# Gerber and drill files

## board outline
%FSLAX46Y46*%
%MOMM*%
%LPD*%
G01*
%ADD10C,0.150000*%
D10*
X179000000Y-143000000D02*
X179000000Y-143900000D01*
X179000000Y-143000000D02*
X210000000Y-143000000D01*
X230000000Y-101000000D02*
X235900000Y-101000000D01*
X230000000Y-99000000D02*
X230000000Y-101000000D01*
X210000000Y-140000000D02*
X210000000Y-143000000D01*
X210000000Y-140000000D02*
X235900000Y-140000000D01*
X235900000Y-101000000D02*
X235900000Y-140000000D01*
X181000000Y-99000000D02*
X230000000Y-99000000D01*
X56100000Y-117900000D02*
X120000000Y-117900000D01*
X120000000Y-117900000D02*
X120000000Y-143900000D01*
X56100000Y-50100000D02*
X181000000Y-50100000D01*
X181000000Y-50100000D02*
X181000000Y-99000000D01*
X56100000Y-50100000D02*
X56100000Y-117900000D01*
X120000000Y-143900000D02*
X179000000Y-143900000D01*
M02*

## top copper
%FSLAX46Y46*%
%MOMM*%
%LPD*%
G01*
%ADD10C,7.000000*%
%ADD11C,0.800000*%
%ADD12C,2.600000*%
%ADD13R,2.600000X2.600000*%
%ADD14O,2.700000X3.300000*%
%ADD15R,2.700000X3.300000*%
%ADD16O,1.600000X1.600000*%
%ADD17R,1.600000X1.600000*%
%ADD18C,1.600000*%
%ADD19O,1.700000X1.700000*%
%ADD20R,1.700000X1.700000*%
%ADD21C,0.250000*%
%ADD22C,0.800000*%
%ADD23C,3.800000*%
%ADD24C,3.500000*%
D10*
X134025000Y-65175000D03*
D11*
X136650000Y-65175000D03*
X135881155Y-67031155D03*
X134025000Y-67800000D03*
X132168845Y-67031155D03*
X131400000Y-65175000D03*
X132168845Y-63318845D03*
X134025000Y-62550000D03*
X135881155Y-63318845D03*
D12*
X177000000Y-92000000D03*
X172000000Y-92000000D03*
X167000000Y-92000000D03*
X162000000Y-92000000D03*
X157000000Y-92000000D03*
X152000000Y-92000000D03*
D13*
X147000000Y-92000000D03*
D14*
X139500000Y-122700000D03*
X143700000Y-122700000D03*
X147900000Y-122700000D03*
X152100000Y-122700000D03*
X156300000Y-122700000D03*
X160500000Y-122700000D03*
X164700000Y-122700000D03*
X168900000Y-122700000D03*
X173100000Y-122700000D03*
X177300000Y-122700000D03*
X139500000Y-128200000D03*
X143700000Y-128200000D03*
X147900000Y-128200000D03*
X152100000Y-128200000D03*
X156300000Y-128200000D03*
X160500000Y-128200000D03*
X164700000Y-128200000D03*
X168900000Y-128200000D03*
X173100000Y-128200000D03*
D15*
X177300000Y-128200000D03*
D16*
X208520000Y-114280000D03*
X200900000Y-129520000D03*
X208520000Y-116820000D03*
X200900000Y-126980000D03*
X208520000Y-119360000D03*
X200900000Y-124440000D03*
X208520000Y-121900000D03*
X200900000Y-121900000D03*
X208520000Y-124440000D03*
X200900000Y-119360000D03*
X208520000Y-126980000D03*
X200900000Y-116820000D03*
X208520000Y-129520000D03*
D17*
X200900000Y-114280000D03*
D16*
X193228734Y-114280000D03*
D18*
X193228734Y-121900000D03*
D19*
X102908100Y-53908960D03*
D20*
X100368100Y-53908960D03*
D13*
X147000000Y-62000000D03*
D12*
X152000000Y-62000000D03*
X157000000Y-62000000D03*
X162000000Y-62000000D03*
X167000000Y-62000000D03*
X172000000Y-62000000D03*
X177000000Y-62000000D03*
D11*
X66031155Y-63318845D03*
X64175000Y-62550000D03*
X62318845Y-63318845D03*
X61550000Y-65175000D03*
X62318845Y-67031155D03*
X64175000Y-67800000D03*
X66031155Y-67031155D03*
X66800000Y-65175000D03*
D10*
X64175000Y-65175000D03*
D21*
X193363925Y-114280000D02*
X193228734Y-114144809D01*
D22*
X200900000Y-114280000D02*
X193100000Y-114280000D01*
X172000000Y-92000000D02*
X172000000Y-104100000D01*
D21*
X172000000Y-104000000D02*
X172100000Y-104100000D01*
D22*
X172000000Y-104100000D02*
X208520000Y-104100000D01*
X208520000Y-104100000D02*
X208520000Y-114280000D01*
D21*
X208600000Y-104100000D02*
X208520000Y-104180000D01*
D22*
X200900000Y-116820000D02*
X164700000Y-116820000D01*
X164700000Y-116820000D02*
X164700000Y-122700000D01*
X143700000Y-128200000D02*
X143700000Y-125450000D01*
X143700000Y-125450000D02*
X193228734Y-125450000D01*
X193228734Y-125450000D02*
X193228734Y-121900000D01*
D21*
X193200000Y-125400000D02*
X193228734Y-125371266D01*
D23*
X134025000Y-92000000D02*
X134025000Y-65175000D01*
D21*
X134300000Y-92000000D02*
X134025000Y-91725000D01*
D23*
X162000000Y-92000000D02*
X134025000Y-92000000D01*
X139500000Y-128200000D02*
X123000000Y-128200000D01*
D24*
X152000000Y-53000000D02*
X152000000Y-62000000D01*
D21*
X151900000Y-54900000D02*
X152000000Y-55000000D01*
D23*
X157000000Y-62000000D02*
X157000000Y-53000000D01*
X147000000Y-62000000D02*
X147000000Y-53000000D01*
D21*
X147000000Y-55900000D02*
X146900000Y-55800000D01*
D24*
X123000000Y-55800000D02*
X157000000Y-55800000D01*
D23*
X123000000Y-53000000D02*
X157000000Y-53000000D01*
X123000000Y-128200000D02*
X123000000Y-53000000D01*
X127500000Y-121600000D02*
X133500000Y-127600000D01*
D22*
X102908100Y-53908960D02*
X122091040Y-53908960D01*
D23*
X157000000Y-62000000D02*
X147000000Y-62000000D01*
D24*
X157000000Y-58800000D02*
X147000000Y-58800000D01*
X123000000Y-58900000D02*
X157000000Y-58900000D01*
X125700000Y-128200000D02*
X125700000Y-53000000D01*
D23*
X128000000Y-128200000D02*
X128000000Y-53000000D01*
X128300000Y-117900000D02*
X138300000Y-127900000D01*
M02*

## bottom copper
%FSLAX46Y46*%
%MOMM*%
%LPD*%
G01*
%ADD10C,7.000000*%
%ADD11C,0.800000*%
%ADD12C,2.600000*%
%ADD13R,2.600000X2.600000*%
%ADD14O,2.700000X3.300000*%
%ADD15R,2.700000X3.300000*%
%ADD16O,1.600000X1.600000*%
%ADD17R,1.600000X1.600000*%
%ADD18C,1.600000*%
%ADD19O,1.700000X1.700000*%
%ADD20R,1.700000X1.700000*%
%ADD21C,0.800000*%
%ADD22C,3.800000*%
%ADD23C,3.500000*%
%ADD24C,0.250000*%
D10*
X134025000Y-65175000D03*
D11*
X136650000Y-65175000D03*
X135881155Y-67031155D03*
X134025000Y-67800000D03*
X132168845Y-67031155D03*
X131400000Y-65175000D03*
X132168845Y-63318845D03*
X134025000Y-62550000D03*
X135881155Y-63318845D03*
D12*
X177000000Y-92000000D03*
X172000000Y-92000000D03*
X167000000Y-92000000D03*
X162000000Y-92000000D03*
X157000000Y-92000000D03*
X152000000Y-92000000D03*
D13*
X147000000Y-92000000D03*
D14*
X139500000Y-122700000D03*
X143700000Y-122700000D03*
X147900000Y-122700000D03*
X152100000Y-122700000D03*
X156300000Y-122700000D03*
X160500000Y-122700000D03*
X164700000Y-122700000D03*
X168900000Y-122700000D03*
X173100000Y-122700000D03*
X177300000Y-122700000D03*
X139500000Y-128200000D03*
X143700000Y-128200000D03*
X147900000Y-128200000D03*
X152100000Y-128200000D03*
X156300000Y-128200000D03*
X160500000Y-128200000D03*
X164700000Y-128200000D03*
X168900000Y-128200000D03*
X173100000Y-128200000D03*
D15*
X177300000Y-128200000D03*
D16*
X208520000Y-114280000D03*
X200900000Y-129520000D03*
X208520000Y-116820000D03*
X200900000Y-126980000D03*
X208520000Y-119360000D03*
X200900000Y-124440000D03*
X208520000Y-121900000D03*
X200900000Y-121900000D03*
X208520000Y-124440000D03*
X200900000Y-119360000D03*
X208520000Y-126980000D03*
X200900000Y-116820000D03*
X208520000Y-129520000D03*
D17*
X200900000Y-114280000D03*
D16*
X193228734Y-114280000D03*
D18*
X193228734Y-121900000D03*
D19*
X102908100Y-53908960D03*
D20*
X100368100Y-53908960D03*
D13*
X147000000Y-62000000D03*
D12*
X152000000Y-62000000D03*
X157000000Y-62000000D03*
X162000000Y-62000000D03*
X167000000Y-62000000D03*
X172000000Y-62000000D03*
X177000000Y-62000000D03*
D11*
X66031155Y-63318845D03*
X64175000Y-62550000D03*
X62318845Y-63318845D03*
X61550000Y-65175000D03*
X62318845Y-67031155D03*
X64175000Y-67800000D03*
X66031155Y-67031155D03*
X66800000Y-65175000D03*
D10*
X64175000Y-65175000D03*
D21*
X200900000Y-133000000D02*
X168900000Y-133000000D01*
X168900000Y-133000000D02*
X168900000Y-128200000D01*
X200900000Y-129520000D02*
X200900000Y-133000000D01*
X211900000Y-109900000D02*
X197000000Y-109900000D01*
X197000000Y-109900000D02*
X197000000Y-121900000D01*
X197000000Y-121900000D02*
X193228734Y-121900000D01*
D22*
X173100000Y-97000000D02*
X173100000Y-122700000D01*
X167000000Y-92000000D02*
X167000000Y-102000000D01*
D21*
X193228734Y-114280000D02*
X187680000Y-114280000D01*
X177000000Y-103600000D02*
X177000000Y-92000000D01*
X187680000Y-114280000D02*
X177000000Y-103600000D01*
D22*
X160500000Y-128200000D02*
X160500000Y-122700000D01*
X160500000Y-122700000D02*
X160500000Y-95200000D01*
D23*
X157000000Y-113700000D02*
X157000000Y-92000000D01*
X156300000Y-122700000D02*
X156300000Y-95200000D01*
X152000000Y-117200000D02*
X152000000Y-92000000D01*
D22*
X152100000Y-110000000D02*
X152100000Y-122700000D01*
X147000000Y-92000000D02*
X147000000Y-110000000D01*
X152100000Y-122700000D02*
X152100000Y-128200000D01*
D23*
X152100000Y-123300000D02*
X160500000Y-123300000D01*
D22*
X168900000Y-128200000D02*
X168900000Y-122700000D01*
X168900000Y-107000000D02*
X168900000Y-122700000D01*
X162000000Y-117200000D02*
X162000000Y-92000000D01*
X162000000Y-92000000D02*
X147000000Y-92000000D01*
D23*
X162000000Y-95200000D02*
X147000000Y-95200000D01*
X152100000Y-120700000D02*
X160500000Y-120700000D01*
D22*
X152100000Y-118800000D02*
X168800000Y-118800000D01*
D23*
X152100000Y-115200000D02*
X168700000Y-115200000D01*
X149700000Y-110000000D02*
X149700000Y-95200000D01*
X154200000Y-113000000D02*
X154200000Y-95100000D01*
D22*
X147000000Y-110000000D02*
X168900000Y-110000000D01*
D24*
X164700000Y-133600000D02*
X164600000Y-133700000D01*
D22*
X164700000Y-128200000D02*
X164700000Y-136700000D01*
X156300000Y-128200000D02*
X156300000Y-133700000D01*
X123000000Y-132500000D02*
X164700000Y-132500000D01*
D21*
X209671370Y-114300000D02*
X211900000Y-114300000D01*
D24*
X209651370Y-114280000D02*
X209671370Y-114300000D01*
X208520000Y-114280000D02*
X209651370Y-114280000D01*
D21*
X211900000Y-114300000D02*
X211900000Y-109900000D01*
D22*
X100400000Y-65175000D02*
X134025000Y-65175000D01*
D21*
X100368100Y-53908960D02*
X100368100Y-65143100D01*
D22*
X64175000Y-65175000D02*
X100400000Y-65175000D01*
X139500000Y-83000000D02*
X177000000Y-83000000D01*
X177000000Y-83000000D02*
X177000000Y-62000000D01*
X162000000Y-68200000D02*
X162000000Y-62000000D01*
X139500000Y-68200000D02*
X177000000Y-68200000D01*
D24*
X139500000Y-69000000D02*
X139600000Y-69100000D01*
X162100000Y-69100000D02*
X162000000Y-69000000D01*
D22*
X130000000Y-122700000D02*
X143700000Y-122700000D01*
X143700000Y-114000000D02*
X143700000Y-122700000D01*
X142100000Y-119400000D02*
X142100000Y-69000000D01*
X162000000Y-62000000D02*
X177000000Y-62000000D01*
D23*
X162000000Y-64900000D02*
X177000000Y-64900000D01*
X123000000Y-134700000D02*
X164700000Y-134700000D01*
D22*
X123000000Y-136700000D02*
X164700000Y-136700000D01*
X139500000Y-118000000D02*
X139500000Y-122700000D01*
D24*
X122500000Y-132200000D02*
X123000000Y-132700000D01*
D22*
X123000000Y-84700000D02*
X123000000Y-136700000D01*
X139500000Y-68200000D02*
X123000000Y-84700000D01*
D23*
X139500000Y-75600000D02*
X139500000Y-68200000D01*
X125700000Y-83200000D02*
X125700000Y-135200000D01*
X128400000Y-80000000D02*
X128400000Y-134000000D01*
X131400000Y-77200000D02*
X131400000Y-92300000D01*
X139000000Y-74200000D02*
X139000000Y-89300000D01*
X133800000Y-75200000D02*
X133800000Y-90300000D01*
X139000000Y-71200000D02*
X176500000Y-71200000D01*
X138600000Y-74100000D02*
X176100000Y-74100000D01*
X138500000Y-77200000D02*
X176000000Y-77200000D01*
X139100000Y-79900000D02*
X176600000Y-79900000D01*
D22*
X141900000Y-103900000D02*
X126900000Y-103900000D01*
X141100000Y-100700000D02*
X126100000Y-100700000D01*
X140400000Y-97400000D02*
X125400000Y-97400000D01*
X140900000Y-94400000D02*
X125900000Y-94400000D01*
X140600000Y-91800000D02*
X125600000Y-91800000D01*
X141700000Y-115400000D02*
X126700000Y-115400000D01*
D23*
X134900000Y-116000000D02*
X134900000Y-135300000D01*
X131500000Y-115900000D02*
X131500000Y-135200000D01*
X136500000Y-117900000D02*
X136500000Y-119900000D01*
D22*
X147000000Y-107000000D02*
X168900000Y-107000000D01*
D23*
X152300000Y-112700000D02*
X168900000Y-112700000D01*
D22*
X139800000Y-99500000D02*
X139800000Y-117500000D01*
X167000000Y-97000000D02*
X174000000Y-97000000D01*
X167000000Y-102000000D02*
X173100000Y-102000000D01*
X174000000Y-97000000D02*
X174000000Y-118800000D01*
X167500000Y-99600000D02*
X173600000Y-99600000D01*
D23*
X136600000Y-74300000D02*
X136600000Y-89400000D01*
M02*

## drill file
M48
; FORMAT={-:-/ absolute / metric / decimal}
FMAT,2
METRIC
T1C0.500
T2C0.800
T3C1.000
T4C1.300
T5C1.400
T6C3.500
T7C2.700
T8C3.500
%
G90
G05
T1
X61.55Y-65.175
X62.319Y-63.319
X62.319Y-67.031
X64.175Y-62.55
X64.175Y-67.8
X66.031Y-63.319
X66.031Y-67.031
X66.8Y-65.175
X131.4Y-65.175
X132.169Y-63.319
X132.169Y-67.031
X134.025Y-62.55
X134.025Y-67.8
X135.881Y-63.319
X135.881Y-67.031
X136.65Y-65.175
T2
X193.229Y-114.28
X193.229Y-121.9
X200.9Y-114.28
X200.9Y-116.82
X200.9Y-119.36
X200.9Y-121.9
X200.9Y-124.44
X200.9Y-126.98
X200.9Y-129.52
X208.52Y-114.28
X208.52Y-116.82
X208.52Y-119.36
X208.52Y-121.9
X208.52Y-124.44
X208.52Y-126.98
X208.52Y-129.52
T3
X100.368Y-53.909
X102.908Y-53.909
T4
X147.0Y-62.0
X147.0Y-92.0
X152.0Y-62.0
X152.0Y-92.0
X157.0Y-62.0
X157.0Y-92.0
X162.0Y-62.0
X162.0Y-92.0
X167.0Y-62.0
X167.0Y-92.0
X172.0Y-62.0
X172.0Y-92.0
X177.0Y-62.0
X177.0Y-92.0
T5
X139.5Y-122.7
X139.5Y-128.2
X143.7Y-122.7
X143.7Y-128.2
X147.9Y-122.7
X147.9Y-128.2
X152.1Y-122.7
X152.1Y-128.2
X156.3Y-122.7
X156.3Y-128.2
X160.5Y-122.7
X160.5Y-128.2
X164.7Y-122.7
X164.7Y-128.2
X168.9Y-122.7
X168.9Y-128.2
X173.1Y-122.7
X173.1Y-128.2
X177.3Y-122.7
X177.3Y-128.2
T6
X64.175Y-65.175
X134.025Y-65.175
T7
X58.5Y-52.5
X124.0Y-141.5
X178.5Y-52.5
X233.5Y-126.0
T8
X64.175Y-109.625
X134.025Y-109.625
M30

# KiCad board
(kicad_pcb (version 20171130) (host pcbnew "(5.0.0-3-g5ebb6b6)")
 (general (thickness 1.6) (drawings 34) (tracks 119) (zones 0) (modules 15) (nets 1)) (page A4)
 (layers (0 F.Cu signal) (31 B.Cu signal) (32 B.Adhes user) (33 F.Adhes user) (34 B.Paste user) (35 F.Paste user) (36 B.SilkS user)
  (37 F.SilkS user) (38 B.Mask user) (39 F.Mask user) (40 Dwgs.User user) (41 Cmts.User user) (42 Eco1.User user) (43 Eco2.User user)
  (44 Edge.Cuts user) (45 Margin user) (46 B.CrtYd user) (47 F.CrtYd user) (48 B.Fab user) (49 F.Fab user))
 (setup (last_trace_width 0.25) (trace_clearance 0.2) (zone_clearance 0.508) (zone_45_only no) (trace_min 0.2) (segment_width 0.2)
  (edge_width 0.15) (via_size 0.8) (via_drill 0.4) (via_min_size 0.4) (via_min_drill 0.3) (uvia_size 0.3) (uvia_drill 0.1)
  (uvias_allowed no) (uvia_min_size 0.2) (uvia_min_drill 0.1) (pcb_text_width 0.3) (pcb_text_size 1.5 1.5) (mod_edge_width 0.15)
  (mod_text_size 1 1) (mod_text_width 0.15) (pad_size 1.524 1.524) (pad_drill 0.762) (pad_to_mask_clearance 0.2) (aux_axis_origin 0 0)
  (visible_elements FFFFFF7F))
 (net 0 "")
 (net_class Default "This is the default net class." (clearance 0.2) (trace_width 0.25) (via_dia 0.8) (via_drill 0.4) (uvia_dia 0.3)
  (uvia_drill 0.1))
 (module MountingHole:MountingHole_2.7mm (layer F.Cu) (at 233.5 126)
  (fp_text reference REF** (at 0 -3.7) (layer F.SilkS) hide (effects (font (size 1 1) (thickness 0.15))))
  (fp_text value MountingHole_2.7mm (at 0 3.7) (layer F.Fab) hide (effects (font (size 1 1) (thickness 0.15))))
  (pad 1 np_thru_hole circle (at 0 0) (size 2.7 2.7) (drill 2.7) (layers *.Cu *.Mask)))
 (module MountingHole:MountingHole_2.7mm (layer F.Cu) (at 58.5 52.5)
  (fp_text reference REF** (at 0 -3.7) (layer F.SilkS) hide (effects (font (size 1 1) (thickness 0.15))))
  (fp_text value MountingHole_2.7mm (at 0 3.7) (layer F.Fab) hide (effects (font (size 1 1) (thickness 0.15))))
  (pad 1 np_thru_hole circle (at 0 0) (size 2.7 2.7) (drill 2.7) (layers *.Cu *.Mask)))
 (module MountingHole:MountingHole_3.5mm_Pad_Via (layer F.Cu) (at 134.025 65.175)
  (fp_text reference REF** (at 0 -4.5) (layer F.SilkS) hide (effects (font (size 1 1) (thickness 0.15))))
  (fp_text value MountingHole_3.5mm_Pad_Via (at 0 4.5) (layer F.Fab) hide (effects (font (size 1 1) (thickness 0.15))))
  (pad 1 thru_hole circle (at 0 0) (size 7 7) (drill 3.5) (layers *.Cu *.Mask))
  (pad 1 thru_hole circle (at 2.625 0) (size 0.8 0.8) (drill 0.5) (layers *.Cu *.Mask))
  (pad 1 thru_hole circle (at 1.856155 1.856155) (size 0.8 0.8) (drill 0.5) (layers *.Cu *.Mask))
  (pad 1 thru_hole circle (at 0 2.625) (size 0.8 0.8) (drill 0.5) (layers *.Cu *.Mask))
  (pad 1 thru_hole circle (at -1.856155 1.856155) (size 0.8 0.8) (drill 0.5) (layers *.Cu *.Mask))
  (pad 1 thru_hole circle (at -2.625 0) (size 0.8 0.8) (drill 0.5) (layers *.Cu *.Mask))
  (pad 1 thru_hole circle (at -1.856155 -1.856155) (size 0.8 0.8) (drill 0.5) (layers *.Cu *.Mask))
  (pad 1 thru_hole circle (at 0 -2.625) (size 0.8 0.8) (drill 0.5) (layers *.Cu *.Mask))
  (pad 1 thru_hole circle (at 1.856155 -1.856155) (size 0.8 0.8) (drill 0.5) (layers *.Cu *.Mask)))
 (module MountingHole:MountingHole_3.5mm (layer F.Cu) (at 134.025 109.625)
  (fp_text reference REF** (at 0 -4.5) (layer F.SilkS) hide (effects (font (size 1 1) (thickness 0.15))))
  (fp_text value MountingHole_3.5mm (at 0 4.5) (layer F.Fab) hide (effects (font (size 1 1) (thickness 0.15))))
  (pad 1 np_thru_hole circle (at 0 0) (size 3.5 3.5) (drill 3.5) (layers *.Cu *.Mask)))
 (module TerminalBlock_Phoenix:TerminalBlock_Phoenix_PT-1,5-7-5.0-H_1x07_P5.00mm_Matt (layer F.Cu) (at 147 92)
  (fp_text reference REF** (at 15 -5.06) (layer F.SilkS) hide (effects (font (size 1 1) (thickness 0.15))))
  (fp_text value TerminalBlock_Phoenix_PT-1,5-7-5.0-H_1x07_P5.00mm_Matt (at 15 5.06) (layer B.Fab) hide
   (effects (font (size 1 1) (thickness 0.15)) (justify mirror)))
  (pad 7 thru_hole circle (at 30 0) (size 2.6 2.6) (drill 1.3) (layers *.Cu *.Mask))
  (pad 6 thru_hole circle (at 25 0) (size 2.6 2.6) (drill 1.3) (layers *.Cu *.Mask))
  (pad 5 thru_hole circle (at 20 0) (size 2.6 2.6) (drill 1.3) (layers *.Cu *.Mask))
  (pad 4 thru_hole circle (at 15 0) (size 2.6 2.6) (drill 1.3) (layers *.Cu *.Mask))
  (pad 3 thru_hole circle (at 10 0) (size 2.6 2.6) (drill 1.3) (layers *.Cu *.Mask))
  (pad 2 thru_hole circle (at 5 0) (size 2.6 2.6) (drill 1.3) (layers *.Cu *.Mask))
  (pad 1 thru_hole rect (at 0 0) (size 2.6 2.6) (drill 1.3) (layers *.Cu *.Mask)))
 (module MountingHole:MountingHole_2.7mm (layer F.Cu) (at 124 141.5)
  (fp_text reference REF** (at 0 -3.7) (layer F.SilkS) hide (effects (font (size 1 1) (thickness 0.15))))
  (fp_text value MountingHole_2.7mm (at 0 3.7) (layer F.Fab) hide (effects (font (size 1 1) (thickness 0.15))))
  (pad 1 np_thru_hole circle (at 0 0) (size 2.7 2.7) (drill 2.7) (layers *.Cu *.Mask)))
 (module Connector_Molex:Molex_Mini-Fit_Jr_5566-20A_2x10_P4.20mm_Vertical (layer F.Cu) (at 177.3 128.2 180)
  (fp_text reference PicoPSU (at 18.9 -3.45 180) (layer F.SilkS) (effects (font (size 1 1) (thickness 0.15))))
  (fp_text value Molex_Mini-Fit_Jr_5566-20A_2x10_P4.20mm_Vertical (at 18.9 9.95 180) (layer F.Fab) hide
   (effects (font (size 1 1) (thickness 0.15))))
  (pad 20 thru_hole oval (at 37.8 5.5 180) (size 2.7 3.3) (drill 1.4) (layers *.Cu *.Mask))
  (pad 19 thru_hole oval (at 33.6 5.5 180) (size 2.7 3.3) (drill 1.4) (layers *.Cu *.Mask))
  (pad 18 thru_hole oval (at 29.4 5.5 180) (size 2.7 3.3) (drill 1.4) (layers *.Cu *.Mask))
  (pad 17 thru_hole oval (at 25.2 5.5 180) (size 2.7 3.3) (drill 1.4) (layers *.Cu *.Mask))
  (pad 16 thru_hole oval (at 21 5.5 180) (size 2.7 3.3) (drill 1.4) (layers *.Cu *.Mask))
  (pad 15 thru_hole oval (at 16.8 5.5 180) (size 2.7 3.3) (drill 1.4) (layers *.Cu *.Mask))
  (pad 14 thru_hole oval (at 12.6 5.5 180) (size 2.7 3.3) (drill 1.4) (layers *.Cu *.Mask))
  (pad 13 thru_hole oval (at 8.4 5.5 180) (size 2.7 3.3) (drill 1.4) (layers *.Cu *.Mask))
  (pad 12 thru_hole oval (at 4.2 5.5 180) (size 2.7 3.3) (drill 1.4) (layers *.Cu *.Mask))
  (pad 11 thru_hole oval (at 0 5.5 180) (size 2.7 3.3) (drill 1.4) (layers *.Cu *.Mask))
  (pad 10 thru_hole oval (at 37.8 0 180) (size 2.7 3.3) (drill 1.4) (layers *.Cu *.Mask))
  (pad 9 thru_hole oval (at 33.6 0 180) (size 2.7 3.3) (drill 1.4) (layers *.Cu *.Mask))
  (pad 8 thru_hole oval (at 29.4 0 180) (size 2.7 3.3) (drill 1.4) (layers *.Cu *.Mask))
  (pad 7 thru_hole oval (at 25.2 0 180) (size 2.7 3.3) (drill 1.4) (layers *.Cu *.Mask))
  (pad 6 thru_hole oval (at 21 0 180) (size 2.7 3.3) (drill 1.4) (layers *.Cu *.Mask))
  (pad 5 thru_hole oval (at 16.8 0 180) (size 2.7 3.3) (drill 1.4) (layers *.Cu *.Mask))
  (pad 4 thru_hole oval (at 12.6 0 180) (size 2.7 3.3) (drill 1.4) (layers *.Cu *.Mask))
  (pad 3 thru_hole oval (at 8.4 0 180) (size 2.7 3.3) (drill 1.4) (layers *.Cu *.Mask))
  (pad 2 thru_hole oval (at 4.2 0 180) (size 2.7 3.3) (drill 1.4) (layers *.Cu *.Mask))
  (pad 1 thru_hole rect (at 0 0 180) (size 2.7 3.3) (drill 1.4) (layers *.Cu *.Mask)))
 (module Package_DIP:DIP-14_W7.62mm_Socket (layer F.Cu) (at 200.9 114.28)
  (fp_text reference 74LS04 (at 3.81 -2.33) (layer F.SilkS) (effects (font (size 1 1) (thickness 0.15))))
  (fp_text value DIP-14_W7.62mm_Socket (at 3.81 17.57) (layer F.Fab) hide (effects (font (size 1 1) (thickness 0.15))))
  (pad 14 thru_hole oval (at 7.62 0) (size 1.6 1.6) (drill 0.8) (layers *.Cu *.Mask))
  (pad 7 thru_hole oval (at 0 15.24) (size 1.6 1.6) (drill 0.8) (layers *.Cu *.Mask))
  (pad 13 thru_hole oval (at 7.62 2.54) (size 1.6 1.6) (drill 0.8) (layers *.Cu *.Mask))
  (pad 6 thru_hole oval (at 0 12.7) (size 1.6 1.6) (drill 0.8) (layers *.Cu *.Mask))
  (pad 12 thru_hole oval (at 7.62 5.08) (size 1.6 1.6) (drill 0.8) (layers *.Cu *.Mask))
  (pad 5 thru_hole oval (at 0 10.16) (size 1.6 1.6) (drill 0.8) (layers *.Cu *.Mask))
  (pad 11 thru_hole oval (at 7.62 7.62) (size 1.6 1.6) (drill 0.8) (layers *.Cu *.Mask))
  (pad 4 thru_hole oval (at 0 7.62) (size 1.6 1.6) (drill 0.8) (layers *.Cu *.Mask))
  (pad 10 thru_hole oval (at 7.62 10.16) (size 1.6 1.6) (drill 0.8) (layers *.Cu *.Mask))
  (pad 3 thru_hole oval (at 0 5.08) (size 1.6 1.6) (drill 0.8) (layers *.Cu *.Mask))
  (pad 9 thru_hole oval (at 7.62 12.7) (size 1.6 1.6) (drill 0.8) (layers *.Cu *.Mask))
  (pad 2 thru_hole oval (at 0 2.54) (size 1.6 1.6) (drill 0.8) (layers *.Cu *.Mask))
  (pad 8 thru_hole oval (at 7.62 15.24) (size 1.6 1.6) (drill 0.8) (layers *.Cu *.Mask))
  (pad 1 thru_hole rect (at 0 0) (size 1.6 1.6) (drill 0.8) (layers *.Cu *.Mask)))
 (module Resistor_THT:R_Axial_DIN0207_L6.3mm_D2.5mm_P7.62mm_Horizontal (layer F.Cu) (at 193.228734 121.9 90)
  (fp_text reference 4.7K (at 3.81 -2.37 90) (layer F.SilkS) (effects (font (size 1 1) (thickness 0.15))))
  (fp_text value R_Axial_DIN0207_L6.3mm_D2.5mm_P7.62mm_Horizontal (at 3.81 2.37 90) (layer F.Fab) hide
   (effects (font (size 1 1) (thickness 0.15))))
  (pad 2 thru_hole oval (at 7.62 0 90) (size 1.6 1.6) (drill 0.8) (layers *.Cu *.Mask))
  (pad 1 thru_hole circle (at 0 0 90) (size 1.6 1.6) (drill 0.8) (layers *.Cu *.Mask)))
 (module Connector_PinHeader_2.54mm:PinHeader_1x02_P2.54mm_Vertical (layer F.Cu) (at 100.3681 53.90896 90)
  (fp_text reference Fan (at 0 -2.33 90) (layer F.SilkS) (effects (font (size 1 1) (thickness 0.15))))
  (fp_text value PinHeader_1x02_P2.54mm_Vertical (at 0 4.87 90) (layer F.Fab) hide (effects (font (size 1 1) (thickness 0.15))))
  (pad 2 thru_hole oval (at 0 2.54 90) (size 1.7 1.7) (drill 1) (layers *.Cu *.Mask))
  (pad 1 thru_hole rect (at 0 0 90) (size 1.7 1.7) (drill 1) (layers *.Cu *.Mask)))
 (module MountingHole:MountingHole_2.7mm (layer F.Cu) (at 178.5 52.5)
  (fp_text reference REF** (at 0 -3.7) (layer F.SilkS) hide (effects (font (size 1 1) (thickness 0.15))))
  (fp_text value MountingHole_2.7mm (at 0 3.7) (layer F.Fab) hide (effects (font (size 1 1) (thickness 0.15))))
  (pad 1 np_thru_hole circle (at 0 0) (size 2.7 2.7) (drill 2.7) (layers *.Cu *.Mask)))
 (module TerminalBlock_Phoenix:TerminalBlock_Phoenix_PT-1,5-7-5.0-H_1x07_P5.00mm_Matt (layer F.Cu) (at 147 62)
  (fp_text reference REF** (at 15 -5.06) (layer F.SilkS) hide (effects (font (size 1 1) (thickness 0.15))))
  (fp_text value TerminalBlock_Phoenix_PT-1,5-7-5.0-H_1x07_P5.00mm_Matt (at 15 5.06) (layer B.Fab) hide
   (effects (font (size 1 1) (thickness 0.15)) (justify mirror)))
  (pad 1 thru_hole rect (at 0 0) (size 2.6 2.6) (drill 1.3) (layers *.Cu *.Mask))
  (pad 2 thru_hole circle (at 5 0) (size 2.6 2.6) (drill 1.3) (layers *.Cu *.Mask))
  (pad 3 thru_hole circle (at 10 0) (size 2.6 2.6) (drill 1.3) (layers *.Cu *.Mask))
  (pad 4 thru_hole circle (at 15 0) (size 2.6 2.6) (drill 1.3) (layers *.Cu *.Mask))
  (pad 5 thru_hole circle (at 20 0) (size 2.6 2.6) (drill 1.3) (layers *.Cu *.Mask))
  (pad 6 thru_hole circle (at 25 0) (size 2.6 2.6) (drill 1.3) (layers *.Cu *.Mask))
  (pad 7 thru_hole circle (at 30 0) (size 2.6 2.6) (drill 1.3) (layers *.Cu *.Mask)))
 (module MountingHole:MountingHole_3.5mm (layer F.Cu) (at 64.175 109.625)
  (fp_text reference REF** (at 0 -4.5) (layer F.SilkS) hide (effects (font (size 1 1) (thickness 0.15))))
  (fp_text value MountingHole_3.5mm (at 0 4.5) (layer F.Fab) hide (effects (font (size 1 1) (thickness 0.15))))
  (pad 1 np_thru_hole circle (at 0 0) (size 3.5 3.5) (drill 3.5) (layers *.Cu *.Mask)))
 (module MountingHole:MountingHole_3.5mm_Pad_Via (layer F.Cu) (at 64.175 65.175)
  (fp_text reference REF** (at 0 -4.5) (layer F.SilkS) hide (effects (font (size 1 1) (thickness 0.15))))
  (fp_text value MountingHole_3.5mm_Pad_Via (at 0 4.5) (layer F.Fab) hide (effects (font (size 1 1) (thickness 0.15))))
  (pad 1 thru_hole circle (at 1.856155 -1.856155) (size 0.8 0.8) (drill 0.5) (layers *.Cu *.Mask))
  (pad 1 thru_hole circle (at 0 -2.625) (size 0.8 0.8) (drill 0.5) (layers *.Cu *.Mask))
  (pad 1 thru_hole circle (at -1.856155 -1.856155) (size 0.8 0.8) (drill 0.5) (layers *.Cu *.Mask))
  (pad 1 thru_hole circle (at -2.625 0) (size 0.8 0.8) (drill 0.5) (layers *.Cu *.Mask))
  (pad 1 thru_hole circle (at -1.856155 1.856155) (size 0.8 0.8) (drill 0.5) (layers *.Cu *.Mask))
  (pad 1 thru_hole circle (at 0 2.625) (size 0.8 0.8) (drill 0.5) (layers *.Cu *.Mask))
  (pad 1 thru_hole circle (at 1.856155 1.856155) (size 0.8 0.8) (drill 0.5) (layers *.Cu *.Mask))
  (pad 1 thru_hole circle (at 2.625 0) (size 0.8 0.8) (drill 0.5) (layers *.Cu *.Mask))
  (pad 1 thru_hole circle (at 0 0) (size 7 7) (drill 3.5) (layers *.Cu *.Mask)))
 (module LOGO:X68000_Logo (layer F.Cu) (at 220 120 90)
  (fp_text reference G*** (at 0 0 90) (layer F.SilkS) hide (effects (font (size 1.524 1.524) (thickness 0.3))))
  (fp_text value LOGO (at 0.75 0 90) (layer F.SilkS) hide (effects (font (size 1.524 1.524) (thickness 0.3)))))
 (gr_line (start 179 143) (end 179 143.9) (layer Edge.Cuts) (width 0.15))
 (gr_line (start 179 143) (end 210 143) (layer Edge.Cuts) (width 0.15))
 (gr_line (start 230 101) (end 235.9 101) (layer Edge.Cuts) (width 0.15))
 (gr_line (start 230 99) (end 230 101) (layer Edge.Cuts) (width 0.15))
 (gr_line (start 210 140) (end 210 143) (layer Edge.Cuts) (width 0.15))
 (gr_line (start 210 140) (end 235.9 140) (layer Edge.Cuts) (width 0.15))
 (gr_line (start 235.9 101) (end 235.9 140) (layer Edge.Cuts) (width 0.15))
 (gr_line (start 181 99) (end 230 99) (layer Edge.Cuts) (width 0.15))
 (gr_line (start 56.1 117.9) (end 120 117.9) (layer Edge.Cuts) (width 0.15))
 (gr_line (start 120 117.9) (end 120 143.9) (layer Edge.Cuts) (width 0.15))
 (gr_line (start 56.1 50.1) (end 181 50.1) (layer Edge.Cuts) (width 0.15))
 (gr_line (start 181 50.1) (end 181 99) (layer Edge.Cuts) (width 0.15))
 (gr_line (start 56.1 50.1) (end 56.1 117.9) (layer Edge.Cuts) (width 0.15))
 (gr_line (start 120 143.9) (end 179 143.9) (layer Edge.Cuts) (width 0.15))
 (segment (start 193.363925 114.28) (end 193.228734 114.144809) (width 0.25) (layer F.Cu) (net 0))
 (segment (start 200.9 114.28) (end 193.1 114.28) (width 0.8) (layer F.Cu) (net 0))
 (segment (start 172 92) (end 172 104.1) (width 0.8) (layer F.Cu) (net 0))
 (segment (start 172 104) (end 172.1 104.1) (width 0.25) (layer F.Cu) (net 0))
 (segment (start 172 104.1) (end 208.52 104.1) (width 0.8) (layer F.Cu) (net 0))
 (segment (start 208.52 104.1) (end 208.52 114.28) (width 0.8) (layer F.Cu) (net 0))
 (segment (start 208.6 104.1) (end 208.52 104.18) (width 0.25) (layer F.Cu) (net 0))
 (segment (start 200.9 116.82) (end 164.7 116.82) (width 0.8) (layer F.Cu) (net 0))
 (segment (start 164.7 116.82) (end 164.7 122.7) (width 0.8) (layer F.Cu) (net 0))
 (segment (start 200.9 133) (end 168.9 133) (width 0.8) (layer B.Cu) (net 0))
 (segment (start 168.9 133) (end 168.9 128.2) (width 0.8) (layer B.Cu) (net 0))
 (segment (start 200.9 129.52) (end 200.9 133) (width 0.8) (layer B.Cu) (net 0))
 (segment (start 211.9 109.9) (end 197 109.9) (width 0.8) (layer B.Cu) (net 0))
 (segment (start 197 109.9) (end 197 121.9) (width 0.8) (layer B.Cu) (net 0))
 (segment (start 197 121.9) (end 193.228734 121.9) (width 0.8) (layer B.Cu) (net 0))
 (segment (start 173.1 97) (end 173.1 122.7) (width 3.8) (layer B.Cu) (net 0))
 (segment (start 167 92) (end 167 102) (width 3.8) (layer B.Cu) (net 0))
 (segment (start 193.228734 114.28) (end 187.68 114.28) (width 0.8) (layer B.Cu) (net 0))
 (segment (start 177 103.6) (end 177 92) (width 0.8) (layer B.Cu) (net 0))
 (segment (start 187.68 114.28) (end 177 103.6) (width 0.8) (layer B.Cu) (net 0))
 (segment (start 160.5 128.2) (end 160.5 122.7) (width 3.8) (layer B.Cu) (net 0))
 (segment (start 160.5 122.7) (end 160.5 95.2) (width 3.8) (layer B.Cu) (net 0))
 (segment (start 157 113.7) (end 157 92) (width 3.5) (layer B.Cu) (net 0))
 (segment (start 156.3 122.7) (end 156.3 95.2) (width 3.5) (layer B.Cu) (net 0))
 (segment (start 152 117.2) (end 152 92) (width 3.5) (layer B.Cu) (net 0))
 (segment (start 152.1 110) (end 152.1 122.7) (width 3.8) (layer B.Cu) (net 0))
 (segment (start 147 92) (end 147 110) (width 3.8) (layer B.Cu) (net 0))
 (segment (start 152.1 122.7) (end 152.1 128.2) (width 3.8) (layer B.Cu) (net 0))
 (segment (start 152.1 123.3) (end 160.5 123.3) (width 3.5) (layer B.Cu) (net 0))
 (segment (start 168.9 128.2) (end 168.9 122.7) (width 3.8) (layer B.Cu) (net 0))
 (segment (start 168.9 107) (end 168.9 122.7) (width 3.8) (layer B.Cu) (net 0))
 (segment (start 162 117.2) (end 162 92) (width 3.8) (layer B.Cu) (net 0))
 (segment (start 162 92) (end 147 92) (width 3.8) (layer B.Cu) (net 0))
 (segment (start 162 95.2) (end 147 95.2) (width 3.5) (layer B.Cu) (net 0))
 (segment (start 152.1 120.7) (end 160.5 120.7) (width 3.5) (layer B.Cu) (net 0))
 (segment (start 152.1 118.8) (end 168.8 118.8) (width 3.8) (layer B.Cu) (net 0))
 (segment (start 152.1 115.2) (end 168.7 115.2) (width 3.5) (layer B.Cu) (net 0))
 (segment (start 149.7 110) (end 149.7 95.2) (width 3.5) (layer B.Cu) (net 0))
 (segment (start 154.2 113) (end 154.2 95.1) (width 3.5) (layer B.Cu) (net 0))
 (segment (start 147 110) (end 168.9 110) (width 3.8) (layer B.Cu) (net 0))
 (segment (start 164.7 133.6) (end 164.6 133.7) (width 0.25) (layer B.Cu) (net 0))
 (segment (start 164.7 128.2) (end 164.7 136.7) (width 3.8) (layer B.Cu) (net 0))
 (segment (start 156.3 128.2) (end 156.3 133.7) (width 3.8) (layer B.Cu) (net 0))
 (segment (start 123 132.5) (end 164.7 132.5) (width 3.8) (layer B.Cu) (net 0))
 (segment (start 209.67137 114.3) (end 211.9 114.3) (width 0.8) (layer B.Cu) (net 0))
 (segment (start 209.65137 114.28) (end 209.67137 114.3) (width 0.25) (layer B.Cu) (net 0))
 (segment (start 208.52 114.28) (end 209.65137 114.28) (width 0.25) (layer B.Cu) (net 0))
 (segment (start 211.9 114.3) (end 211.9 109.9) (width 0.8) (layer B.Cu) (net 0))
 (segment (start 143.7 128.2) (end 143.7 125.45) (width 0.8) (layer F.Cu) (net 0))
 (segment (start 143.7 125.45) (end 193.228734 125.45) (width 0.8) (layer F.Cu) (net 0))
 (segment (start 193.228734 125.45) (end 193.228734 121.9) (width 0.8) (layer F.Cu) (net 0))
 (segment (start 193.2 125.4) (end 193.228734 125.371266) (width 0.25) (layer F.Cu) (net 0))
 (segment (start 134.025 92) (end 134.025 65.175) (width 3.8) (layer F.Cu) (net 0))
 (segment (start 134.3 92) (end 134.025 91.725) (width 0.25) (layer F.Cu) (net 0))
 (segment (start 162 92) (end 134.025 92) (width 3.8) (layer F.Cu) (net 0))
 (segment (start 139.5 128.2) (end 123 128.2) (width 3.8) (layer F.Cu) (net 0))
 (segment (start 152 53) (end 152 62) (width 3.5) (layer F.Cu) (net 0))
 (segment (start 151.9 54.9) (end 152 55) (width 0.25) (layer F.Cu) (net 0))
 (segment (start 157 62) (end 157 53) (width 3.8) (layer F.Cu) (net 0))
 (segment (start 147 62) (end 147 53) (width 3.8) (layer F.Cu) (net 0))
 (segment (start 147 55.9) (end 146.9 55.8) (width 0.25) (layer F.Cu) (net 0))
 (segment (start 123 55.8) (end 157 55.8) (width 3.5) (layer F.Cu) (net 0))
 (segment (start 123 53) (end 157 53) (width 3.8) (layer F.Cu) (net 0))
 (segment (start 123 128.2) (end 123 53) (width 3.8) (layer F.Cu) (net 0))
 (segment (start 127.5 121.6) (end 133.5 127.6) (width 3.8) (layer F.Cu) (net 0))
 (segment (start 102.9081 53.90896) (end 122.09104 53.90896) (width 0.8) (layer F.Cu) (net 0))
 (segment (start 100.4 65.175) (end 134.025 65.175) (width 3.8) (layer B.Cu) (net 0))
 (segment (start 100.3681 53.90896) (end 100.3681 65.1431) (width 0.8) (layer B.Cu) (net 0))
 (segment (start 64.175 65.175) (end 100.4 65.175) (width 3.8) (layer B.Cu) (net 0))
 (segment (start 139.5 83) (end 177 83) (width 3.8) (layer B.Cu) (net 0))
 (segment (start 177 83) (end 177 62) (width 3.8) (layer B.Cu) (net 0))
 (segment (start 162 68.2) (end 162 62) (width 3.8) (layer B.Cu) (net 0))
 (segment (start 139.5 68.2) (end 177 68.2) (width 3.8) (layer B.Cu) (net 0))
 (segment (start 139.5 69) (end 139.6 69.1) (width 0.25) (layer B.Cu) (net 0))
 (segment (start 162.1 69.1) (end 162 69) (width 0.25) (layer B.Cu) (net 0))
 (segment (start 130 122.7) (end 143.7 122.7) (width 3.8) (layer B.Cu) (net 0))
 (segment (start 143.7 114) (end 143.7 122.7) (width 3.8) (layer B.Cu) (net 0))
 (segment (start 142.1 119.4) (end 142.1 69) (width 3.8) (layer B.Cu) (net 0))
 (segment (start 162 62) (end 177 62) (width 3.8) (layer B.Cu) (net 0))
 (segment (start 162 64.9) (end 177 64.9) (width 3.5) (layer B.Cu) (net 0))
 (segment (start 157 62) (end 147 62) (width 3.8) (layer F.Cu) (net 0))
 (segment (start 157 58.8) (end 147 58.8) (width 3.5) (layer F.Cu) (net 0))
 (segment (start 123 134.7) (end 164.7 134.7) (width 3.5) (layer B.Cu) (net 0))
 (segment (start 123 136.7) (end 164.7 136.7) (width 3.8) (layer B.Cu) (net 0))
 (segment (start 139.5 118) (end 139.5 122.7) (width 3.8) (layer B.Cu) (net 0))
 (segment (start 122.5 132.2) (end 123 132.7) (width 0.25) (layer B.Cu) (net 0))
 (segment (start 123 84.7) (end 123 136.7) (width 3.8) (layer B.Cu) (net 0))
 (segment (start 139.5 68.2) (end 123 84.7) (width 3.8) (layer B.Cu) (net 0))
 (segment (start 139.5 75.6) (end 139.5 68.2) (width 3.5) (layer B.Cu) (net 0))
 (segment (start 125.7 83.2) (end 125.7 135.2) (width 3.5) (layer B.Cu) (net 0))
 (segment (start 128.4 80) (end 128.4 134) (width 3.5) (layer B.Cu) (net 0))
 (segment (start 131.4 77.2) (end 131.4 92.3) (width 3.5) (layer B.Cu) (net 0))
 (segment (start 139 74.2) (end 139 89.3) (width 3.5) (layer B.Cu) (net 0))
 (segment (start 133.8 75.2) (end 133.8 90.3) (width 3.5) (layer B.Cu) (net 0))
 (segment (start 139 71.2) (end 176.5 71.2) (width 3.5) (layer B.Cu) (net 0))
 (segment (start 138.6 74.1) (end 176.1 74.1) (width 3.5) (layer B.Cu) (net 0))
 (segment (start 138.5 77.2) (end 176 77.2) (width 3.5) (layer B.Cu) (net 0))
 (segment (start 139.1 79.9) (end 176.6 79.9) (width 3.5) (layer B.Cu) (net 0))
 (segment (start 141.9 103.9) (end 126.9 103.9) (width 3.8) (layer B.Cu) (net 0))
 (segment (start 141.1 100.7) (end 126.1 100.7) (width 3.8) (layer B.Cu) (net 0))
 (segment (start 140.4 97.4) (end 125.4 97.4) (width 3.8) (layer B.Cu) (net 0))
 (segment (start 140.9 94.4) (end 125.9 94.4) (width 3.8) (layer B.Cu) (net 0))
 (segment (start 140.6 91.8) (end 125.6 91.8) (width 3.8) (layer B.Cu) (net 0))
 (segment (start 141.7 115.4) (end 126.7 115.4) (width 3.8) (layer B.Cu) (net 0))
 (segment (start 134.9 116) (end 134.9 135.3) (width 3.5) (layer B.Cu) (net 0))
 (segment (start 131.5 115.9) (end 131.5 135.2) (width 3.5) (layer B.Cu) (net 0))
 (segment (start 136.5 117.9) (end 136.5 119.9) (width 3.5) (layer B.Cu) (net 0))
 (segment (start 147 107) (end 168.9 107) (width 3.8) (layer B.Cu) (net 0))
 (segment (start 152.3 112.7) (end 168.9 112.7) (width 3.5) (layer B.Cu) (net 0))
 (segment (start 139.8 99.5) (end 139.8 117.5) (width 3.8) (layer B.Cu) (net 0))
 (segment (start 167 97) (end 174 97) (width 3.8) (layer B.Cu) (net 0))
 (segment (start 167 102) (end 173.1 102) (width 3.8) (layer B.Cu) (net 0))
 (segment (start 174 97) (end 174 118.8) (width 3.8) (layer B.Cu) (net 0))
 (segment (start 167.5 99.6) (end 173.6 99.6) (width 3.8) (layer B.Cu) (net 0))
 (segment (start 136.6 74.3) (end 136.6 89.4) (width 3.5) (layer B.Cu) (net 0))
 (segment (start 123 58.9) (end 157 58.9) (width 3.5) (layer F.Cu) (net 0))
 (segment (start 125.7 128.2) (end 125.7 53) (width 3.5) (layer F.Cu) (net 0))
 (segment (start 128 128.2) (end 128 53) (width 3.8) (layer F.Cu) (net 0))
 (segment (start 128.3 117.9) (end 138.3 127.9) (width 3.8) (layer F.Cu) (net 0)))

